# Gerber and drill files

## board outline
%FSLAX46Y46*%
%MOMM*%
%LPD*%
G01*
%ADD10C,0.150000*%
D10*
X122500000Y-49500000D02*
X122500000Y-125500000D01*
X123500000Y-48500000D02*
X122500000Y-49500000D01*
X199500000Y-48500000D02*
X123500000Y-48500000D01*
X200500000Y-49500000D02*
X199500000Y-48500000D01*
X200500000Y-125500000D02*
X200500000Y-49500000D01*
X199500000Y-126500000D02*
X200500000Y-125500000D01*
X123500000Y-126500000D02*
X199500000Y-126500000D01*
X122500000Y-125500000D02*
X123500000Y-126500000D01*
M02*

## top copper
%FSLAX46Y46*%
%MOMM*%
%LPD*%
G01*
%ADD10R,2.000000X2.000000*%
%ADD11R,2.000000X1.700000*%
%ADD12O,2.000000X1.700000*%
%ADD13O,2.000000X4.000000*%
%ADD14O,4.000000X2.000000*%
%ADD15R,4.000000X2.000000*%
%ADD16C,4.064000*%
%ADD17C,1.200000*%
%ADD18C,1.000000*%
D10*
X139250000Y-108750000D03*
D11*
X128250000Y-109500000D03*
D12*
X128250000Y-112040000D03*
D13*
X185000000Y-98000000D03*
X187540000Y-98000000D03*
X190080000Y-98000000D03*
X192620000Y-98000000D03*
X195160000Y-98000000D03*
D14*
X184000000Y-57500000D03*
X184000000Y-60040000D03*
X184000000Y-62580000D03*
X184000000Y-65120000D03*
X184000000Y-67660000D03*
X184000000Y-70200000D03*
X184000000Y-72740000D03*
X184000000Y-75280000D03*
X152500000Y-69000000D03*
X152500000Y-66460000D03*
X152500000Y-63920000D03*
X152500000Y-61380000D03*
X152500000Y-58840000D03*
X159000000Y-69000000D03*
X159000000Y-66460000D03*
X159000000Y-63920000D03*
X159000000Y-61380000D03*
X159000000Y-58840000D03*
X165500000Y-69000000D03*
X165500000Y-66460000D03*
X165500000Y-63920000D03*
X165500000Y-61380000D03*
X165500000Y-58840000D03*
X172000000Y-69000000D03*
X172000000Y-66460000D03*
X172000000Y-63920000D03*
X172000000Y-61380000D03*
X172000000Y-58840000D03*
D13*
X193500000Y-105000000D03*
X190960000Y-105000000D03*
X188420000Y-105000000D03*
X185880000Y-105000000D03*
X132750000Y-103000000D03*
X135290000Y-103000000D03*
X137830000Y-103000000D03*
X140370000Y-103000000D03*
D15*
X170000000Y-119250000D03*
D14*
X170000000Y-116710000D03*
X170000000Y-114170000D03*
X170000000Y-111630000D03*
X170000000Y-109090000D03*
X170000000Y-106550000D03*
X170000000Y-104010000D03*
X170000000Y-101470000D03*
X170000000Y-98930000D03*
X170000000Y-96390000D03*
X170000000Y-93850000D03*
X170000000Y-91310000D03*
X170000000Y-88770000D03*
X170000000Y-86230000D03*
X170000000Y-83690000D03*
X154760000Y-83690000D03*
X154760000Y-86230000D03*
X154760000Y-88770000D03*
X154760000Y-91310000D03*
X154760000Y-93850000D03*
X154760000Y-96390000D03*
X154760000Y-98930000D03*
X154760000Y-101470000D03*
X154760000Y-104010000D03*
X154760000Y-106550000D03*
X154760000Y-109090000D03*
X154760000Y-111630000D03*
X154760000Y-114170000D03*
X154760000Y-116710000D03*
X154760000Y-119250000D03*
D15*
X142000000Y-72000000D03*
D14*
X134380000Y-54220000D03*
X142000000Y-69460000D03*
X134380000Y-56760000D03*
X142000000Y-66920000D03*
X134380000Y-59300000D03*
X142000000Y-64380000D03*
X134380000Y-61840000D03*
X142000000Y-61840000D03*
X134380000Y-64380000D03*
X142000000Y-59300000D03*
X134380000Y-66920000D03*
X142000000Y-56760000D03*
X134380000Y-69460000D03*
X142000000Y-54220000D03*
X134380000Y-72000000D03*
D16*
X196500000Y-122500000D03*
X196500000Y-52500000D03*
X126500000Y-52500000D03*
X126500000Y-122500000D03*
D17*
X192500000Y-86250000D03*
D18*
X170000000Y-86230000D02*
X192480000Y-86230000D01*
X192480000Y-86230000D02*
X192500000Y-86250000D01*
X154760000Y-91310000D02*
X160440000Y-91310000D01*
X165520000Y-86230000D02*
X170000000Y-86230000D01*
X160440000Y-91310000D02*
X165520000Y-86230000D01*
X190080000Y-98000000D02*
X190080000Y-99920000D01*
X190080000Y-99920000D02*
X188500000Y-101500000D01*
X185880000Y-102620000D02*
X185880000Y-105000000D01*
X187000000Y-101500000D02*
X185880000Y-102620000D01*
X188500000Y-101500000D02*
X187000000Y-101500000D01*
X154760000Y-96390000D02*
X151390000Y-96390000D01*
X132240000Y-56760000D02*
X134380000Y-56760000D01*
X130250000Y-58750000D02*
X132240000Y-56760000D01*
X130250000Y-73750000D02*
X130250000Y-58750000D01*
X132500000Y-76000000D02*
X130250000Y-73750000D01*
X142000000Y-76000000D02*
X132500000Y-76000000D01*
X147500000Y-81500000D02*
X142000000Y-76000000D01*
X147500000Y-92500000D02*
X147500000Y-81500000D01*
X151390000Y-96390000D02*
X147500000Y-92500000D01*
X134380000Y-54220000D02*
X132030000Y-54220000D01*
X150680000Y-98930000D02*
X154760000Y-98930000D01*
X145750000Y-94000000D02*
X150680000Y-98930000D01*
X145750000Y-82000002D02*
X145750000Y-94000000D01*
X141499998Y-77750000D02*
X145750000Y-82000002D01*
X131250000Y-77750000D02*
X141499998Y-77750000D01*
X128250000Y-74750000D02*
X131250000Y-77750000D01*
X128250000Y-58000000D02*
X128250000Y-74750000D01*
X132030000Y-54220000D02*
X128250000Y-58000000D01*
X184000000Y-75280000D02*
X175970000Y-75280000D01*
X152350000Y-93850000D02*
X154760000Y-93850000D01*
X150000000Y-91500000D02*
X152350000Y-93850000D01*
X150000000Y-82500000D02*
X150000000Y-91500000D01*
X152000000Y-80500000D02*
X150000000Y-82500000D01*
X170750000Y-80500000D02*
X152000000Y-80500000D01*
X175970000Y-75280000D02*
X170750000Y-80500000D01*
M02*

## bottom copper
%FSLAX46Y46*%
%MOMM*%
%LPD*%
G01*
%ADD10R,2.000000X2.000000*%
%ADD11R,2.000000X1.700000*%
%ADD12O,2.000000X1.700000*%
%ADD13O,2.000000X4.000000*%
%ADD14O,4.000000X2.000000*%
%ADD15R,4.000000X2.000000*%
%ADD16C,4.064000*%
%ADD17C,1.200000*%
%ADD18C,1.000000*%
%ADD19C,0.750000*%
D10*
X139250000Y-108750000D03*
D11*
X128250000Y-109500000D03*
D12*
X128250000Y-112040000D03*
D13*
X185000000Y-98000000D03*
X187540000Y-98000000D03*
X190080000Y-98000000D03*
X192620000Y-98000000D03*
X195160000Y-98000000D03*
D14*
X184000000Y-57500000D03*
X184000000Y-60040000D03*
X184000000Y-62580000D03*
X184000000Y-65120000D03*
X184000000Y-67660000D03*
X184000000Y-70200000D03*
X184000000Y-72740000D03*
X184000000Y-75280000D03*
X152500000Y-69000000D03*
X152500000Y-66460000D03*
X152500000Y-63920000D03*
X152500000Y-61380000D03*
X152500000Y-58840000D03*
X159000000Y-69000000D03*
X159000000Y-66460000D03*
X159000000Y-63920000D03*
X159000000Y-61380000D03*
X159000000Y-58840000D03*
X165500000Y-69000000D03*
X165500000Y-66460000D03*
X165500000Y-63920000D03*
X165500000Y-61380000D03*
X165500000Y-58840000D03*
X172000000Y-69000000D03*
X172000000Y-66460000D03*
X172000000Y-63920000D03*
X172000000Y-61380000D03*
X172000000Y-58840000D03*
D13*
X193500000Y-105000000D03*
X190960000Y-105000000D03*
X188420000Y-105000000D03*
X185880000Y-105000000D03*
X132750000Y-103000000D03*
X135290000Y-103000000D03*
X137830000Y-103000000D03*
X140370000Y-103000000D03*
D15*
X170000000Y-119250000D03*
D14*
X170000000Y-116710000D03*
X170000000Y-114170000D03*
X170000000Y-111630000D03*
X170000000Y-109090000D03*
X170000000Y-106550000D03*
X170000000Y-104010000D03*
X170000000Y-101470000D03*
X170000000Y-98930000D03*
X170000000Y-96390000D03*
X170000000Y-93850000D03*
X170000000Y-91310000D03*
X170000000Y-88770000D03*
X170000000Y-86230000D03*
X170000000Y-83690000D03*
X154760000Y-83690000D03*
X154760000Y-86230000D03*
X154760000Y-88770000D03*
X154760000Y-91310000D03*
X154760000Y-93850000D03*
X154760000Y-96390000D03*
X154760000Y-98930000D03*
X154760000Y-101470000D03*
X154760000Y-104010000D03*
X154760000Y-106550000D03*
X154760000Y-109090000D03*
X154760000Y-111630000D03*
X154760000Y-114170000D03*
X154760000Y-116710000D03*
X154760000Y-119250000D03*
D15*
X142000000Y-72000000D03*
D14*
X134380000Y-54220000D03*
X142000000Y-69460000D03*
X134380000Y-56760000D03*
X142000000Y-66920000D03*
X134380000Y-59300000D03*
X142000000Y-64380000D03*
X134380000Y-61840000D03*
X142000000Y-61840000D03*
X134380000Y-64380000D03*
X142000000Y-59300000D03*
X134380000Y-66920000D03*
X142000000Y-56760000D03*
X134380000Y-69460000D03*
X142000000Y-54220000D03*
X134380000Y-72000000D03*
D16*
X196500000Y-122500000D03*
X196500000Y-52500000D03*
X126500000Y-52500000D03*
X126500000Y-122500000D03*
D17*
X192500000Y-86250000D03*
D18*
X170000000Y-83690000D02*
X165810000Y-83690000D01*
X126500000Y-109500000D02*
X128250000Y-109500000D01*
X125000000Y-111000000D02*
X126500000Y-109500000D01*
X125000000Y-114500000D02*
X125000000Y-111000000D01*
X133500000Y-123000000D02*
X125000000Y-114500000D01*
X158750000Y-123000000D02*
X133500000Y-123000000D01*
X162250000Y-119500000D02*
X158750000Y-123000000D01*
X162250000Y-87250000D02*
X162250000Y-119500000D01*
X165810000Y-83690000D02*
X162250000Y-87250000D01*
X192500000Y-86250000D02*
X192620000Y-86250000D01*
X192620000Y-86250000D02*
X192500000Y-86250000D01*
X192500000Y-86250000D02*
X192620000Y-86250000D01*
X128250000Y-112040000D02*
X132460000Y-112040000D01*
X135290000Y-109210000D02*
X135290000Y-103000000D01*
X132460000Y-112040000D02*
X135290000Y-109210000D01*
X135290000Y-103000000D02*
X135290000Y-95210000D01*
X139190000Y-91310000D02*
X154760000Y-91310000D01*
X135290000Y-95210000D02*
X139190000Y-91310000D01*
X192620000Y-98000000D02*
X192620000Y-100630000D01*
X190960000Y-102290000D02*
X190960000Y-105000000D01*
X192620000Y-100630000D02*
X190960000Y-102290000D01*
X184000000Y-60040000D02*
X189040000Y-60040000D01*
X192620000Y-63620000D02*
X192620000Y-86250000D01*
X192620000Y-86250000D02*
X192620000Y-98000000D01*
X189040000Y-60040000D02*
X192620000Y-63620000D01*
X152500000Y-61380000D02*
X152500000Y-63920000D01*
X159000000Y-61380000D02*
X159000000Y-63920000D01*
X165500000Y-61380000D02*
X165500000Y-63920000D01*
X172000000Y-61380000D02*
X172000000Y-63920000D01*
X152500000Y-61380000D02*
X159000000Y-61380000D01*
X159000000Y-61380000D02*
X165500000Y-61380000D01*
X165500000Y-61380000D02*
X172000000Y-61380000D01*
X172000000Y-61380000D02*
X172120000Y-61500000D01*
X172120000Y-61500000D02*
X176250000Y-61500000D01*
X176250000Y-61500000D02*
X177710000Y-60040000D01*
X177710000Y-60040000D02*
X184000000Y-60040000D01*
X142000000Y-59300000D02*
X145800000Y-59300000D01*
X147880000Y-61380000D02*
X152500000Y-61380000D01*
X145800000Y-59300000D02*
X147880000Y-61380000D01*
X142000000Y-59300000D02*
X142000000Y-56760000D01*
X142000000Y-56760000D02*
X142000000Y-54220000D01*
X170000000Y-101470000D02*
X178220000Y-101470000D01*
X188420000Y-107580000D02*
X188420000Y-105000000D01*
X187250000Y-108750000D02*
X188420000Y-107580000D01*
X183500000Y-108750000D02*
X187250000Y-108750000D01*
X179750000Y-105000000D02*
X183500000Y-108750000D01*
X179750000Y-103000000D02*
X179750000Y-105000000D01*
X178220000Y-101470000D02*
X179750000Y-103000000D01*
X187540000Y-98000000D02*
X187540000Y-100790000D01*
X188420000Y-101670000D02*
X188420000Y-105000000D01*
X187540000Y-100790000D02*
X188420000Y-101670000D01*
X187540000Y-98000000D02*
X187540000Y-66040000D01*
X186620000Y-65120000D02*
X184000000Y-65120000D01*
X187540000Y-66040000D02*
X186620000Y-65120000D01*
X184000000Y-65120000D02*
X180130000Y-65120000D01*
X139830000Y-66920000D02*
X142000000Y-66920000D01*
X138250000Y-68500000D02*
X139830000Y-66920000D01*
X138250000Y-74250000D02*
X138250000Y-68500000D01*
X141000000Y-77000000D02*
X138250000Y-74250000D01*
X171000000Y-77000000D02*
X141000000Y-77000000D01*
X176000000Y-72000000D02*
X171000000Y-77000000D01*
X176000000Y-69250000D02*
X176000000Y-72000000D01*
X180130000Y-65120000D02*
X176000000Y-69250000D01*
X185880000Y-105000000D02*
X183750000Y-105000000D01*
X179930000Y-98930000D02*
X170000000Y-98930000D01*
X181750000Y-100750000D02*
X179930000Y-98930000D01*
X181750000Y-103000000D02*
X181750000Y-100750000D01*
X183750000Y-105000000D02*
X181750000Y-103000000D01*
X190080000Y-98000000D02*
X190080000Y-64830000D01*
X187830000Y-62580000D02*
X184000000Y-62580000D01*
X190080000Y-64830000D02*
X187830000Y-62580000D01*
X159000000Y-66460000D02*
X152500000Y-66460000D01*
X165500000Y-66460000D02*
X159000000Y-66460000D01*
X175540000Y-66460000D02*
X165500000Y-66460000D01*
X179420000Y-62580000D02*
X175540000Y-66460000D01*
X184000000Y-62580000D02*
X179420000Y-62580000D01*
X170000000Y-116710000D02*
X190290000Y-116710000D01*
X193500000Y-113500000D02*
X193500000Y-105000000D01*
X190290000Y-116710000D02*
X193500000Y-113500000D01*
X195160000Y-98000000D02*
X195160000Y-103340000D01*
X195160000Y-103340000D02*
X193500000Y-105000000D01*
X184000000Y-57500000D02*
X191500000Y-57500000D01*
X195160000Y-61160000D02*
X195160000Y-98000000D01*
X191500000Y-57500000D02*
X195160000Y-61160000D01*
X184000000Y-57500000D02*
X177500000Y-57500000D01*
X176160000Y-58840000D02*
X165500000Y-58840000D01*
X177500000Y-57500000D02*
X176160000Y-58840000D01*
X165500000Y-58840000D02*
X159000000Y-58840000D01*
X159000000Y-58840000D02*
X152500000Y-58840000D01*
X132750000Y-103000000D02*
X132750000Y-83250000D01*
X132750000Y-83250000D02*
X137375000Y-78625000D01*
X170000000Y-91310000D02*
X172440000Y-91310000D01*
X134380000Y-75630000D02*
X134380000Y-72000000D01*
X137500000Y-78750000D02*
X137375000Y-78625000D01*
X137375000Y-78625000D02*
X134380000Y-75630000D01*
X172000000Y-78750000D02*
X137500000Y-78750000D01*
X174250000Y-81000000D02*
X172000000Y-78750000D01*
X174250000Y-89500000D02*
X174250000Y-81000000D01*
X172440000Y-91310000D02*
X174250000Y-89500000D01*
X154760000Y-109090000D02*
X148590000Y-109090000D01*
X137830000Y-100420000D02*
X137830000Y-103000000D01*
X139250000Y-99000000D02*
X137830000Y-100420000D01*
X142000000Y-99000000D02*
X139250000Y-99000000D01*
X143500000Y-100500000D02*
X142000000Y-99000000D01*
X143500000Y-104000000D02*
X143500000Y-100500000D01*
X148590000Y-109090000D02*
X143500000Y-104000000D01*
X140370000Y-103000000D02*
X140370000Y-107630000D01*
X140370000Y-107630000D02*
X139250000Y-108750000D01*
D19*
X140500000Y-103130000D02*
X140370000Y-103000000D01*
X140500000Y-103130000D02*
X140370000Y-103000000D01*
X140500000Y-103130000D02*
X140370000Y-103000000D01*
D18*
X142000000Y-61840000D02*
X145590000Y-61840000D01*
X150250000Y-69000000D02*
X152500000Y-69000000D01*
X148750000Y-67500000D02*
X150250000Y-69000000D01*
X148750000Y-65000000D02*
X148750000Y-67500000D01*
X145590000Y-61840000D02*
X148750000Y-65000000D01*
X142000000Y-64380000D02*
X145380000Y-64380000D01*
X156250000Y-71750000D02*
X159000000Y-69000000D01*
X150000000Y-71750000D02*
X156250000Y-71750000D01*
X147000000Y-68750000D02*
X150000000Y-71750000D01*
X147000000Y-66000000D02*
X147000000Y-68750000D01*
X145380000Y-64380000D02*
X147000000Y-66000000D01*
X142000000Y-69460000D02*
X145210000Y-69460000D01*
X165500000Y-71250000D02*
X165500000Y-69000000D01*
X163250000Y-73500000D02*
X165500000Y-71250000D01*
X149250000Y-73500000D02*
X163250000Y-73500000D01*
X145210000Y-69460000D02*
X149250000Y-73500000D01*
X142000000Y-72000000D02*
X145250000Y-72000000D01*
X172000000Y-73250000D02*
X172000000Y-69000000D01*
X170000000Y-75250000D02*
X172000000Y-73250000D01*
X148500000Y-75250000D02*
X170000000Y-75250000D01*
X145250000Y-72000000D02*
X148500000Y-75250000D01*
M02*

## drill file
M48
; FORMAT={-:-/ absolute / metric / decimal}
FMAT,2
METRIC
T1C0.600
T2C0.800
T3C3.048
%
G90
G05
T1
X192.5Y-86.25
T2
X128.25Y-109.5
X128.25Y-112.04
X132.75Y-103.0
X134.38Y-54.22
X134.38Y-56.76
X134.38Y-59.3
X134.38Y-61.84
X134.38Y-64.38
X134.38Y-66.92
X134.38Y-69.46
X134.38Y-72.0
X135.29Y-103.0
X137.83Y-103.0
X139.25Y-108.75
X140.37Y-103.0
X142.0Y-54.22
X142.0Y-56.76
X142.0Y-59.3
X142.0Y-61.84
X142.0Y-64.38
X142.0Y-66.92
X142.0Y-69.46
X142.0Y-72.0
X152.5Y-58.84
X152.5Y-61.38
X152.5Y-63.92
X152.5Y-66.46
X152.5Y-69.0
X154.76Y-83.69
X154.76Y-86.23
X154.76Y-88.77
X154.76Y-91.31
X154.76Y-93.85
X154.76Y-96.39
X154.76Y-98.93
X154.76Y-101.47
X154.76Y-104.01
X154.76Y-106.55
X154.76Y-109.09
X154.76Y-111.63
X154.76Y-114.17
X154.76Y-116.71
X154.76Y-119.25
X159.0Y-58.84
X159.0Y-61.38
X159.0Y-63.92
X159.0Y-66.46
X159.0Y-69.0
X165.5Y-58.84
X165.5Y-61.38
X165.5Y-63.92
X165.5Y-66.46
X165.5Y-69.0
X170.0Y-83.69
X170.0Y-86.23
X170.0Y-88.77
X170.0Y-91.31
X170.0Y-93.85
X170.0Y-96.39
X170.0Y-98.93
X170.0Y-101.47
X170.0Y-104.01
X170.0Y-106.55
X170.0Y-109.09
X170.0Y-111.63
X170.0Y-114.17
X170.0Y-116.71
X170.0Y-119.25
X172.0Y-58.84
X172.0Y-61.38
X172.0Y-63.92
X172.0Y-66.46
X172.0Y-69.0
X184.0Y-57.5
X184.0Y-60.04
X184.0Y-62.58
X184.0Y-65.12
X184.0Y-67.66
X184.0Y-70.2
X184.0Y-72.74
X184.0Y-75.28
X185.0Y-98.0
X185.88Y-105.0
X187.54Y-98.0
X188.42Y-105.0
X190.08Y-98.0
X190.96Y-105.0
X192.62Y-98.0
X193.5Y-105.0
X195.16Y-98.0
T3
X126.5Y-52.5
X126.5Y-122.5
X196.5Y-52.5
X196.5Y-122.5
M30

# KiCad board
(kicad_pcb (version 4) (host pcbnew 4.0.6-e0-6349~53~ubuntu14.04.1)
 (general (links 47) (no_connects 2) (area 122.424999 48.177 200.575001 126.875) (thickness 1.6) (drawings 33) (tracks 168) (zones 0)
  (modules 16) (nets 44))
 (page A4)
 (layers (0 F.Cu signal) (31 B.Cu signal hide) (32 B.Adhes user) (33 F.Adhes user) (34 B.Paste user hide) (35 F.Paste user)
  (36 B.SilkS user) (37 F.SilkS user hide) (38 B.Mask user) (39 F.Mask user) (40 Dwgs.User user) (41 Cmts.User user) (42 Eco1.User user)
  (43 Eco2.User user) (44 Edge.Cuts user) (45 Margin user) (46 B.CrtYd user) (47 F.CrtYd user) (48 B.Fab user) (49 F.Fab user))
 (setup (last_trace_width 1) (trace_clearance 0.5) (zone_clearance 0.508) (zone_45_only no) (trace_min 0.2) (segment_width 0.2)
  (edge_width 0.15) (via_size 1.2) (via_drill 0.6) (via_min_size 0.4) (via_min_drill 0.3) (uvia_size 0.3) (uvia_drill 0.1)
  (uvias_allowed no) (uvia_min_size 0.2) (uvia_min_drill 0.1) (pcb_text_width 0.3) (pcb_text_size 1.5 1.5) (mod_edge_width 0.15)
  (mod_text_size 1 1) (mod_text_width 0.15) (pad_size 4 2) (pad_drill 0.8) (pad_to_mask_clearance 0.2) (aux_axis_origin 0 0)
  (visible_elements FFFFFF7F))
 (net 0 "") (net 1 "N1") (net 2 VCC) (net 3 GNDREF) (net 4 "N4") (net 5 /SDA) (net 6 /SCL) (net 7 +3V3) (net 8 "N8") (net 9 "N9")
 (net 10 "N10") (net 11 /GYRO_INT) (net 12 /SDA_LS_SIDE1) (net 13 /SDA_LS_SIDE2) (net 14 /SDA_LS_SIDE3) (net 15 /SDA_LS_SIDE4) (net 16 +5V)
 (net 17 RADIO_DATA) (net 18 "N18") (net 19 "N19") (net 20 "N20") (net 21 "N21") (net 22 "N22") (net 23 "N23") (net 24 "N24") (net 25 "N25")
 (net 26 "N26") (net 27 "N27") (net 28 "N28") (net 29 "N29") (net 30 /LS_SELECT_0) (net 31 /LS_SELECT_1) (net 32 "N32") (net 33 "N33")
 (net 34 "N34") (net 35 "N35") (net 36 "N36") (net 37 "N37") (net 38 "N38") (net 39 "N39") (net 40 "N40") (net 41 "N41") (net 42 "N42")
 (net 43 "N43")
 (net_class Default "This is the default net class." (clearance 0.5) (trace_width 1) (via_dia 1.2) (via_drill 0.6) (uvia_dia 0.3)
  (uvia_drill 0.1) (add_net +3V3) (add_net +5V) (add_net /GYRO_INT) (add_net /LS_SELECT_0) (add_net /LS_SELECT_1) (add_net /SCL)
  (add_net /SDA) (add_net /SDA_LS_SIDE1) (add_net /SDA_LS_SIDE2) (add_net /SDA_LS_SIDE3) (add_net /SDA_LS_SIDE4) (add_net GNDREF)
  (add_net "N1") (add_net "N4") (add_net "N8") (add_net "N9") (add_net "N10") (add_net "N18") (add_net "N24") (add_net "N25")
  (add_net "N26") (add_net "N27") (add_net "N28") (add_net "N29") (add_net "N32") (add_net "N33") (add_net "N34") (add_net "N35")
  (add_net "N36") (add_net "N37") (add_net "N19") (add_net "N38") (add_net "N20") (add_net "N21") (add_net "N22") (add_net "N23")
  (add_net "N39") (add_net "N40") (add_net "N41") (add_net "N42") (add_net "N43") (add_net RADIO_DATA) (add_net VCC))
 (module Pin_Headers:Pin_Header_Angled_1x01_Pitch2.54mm (layer F.Cu) (at 139.25 108.75 270)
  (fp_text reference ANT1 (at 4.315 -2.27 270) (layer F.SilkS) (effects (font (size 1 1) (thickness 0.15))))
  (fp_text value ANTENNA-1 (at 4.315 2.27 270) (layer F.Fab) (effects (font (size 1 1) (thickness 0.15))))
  (pad 1 thru_hole rect (at 0 0 270) (size 2 2) (drill 0.8) (layers *.Cu *.Mask) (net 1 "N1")))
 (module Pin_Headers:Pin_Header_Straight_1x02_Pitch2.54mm (layer F.Cu) (at 128.25 109.5)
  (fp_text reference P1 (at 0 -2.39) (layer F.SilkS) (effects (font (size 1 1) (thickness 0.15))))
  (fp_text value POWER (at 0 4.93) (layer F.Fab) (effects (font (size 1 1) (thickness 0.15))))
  (pad 1 thru_hole rect (at 0 0) (size 2 1.7) (drill 0.8) (layers *.Cu *.Mask) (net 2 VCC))
  (pad 2 thru_hole oval (at 0 2.54) (size 2 1.7) (drill 0.8) (layers *.Cu *.Mask) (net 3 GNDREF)))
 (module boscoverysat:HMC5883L (layer F.Cu) (at 185 98)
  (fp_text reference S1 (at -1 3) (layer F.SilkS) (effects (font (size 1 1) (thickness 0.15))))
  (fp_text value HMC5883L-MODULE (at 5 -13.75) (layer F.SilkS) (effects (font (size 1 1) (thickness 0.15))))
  (pad 1 thru_hole oval (at 0 0) (size 2 4) (drill 0.8) (layers *.Cu F.SilkS B.Mask) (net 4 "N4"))
  (pad 2 thru_hole oval (at 2.54 0) (size 2 4) (drill 0.8) (layers *.Cu F.SilkS B.Mask) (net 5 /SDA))
  (pad 3 thru_hole oval (at 5.08 0) (size 2 4) (drill 0.8) (layers *.Cu F.SilkS B.Mask) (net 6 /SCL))
  (pad 4 thru_hole oval (at 7.62 0) (size 2 4) (drill 0.8) (layers *.Cu F.SilkS B.Mask) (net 3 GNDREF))
  (pad 5 thru_hole oval (at 10.16 0) (size 2 4) (drill 0.8) (layers *.Cu F.SilkS B.Mask) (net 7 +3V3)))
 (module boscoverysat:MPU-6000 (layer F.Cu) (at 184 57.5 270)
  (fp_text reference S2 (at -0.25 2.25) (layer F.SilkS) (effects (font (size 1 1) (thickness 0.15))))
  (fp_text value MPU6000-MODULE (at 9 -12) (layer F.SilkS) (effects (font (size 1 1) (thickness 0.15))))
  (pad 1 thru_hole oval (at 0 0 270) (size 2 4) (drill 0.8) (layers *.Cu F.SilkS B.Mask) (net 7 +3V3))
  (pad 2 thru_hole oval (at 2.54 0 270) (size 2 4) (drill 0.8) (layers *.Cu F.SilkS B.Mask) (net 3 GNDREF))
  (pad 3 thru_hole oval (at 5.08 0 270) (size 2 4) (drill 0.8) (layers *.Cu F.SilkS B.Mask) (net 6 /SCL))
  (pad 4 thru_hole oval (at 7.62 0 270) (size 2 4) (drill 0.8) (layers *.Cu F.SilkS B.Mask) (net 5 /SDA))
  (pad 5 thru_hole oval (at 10.16 0 270) (size 2 4) (drill 0.8) (layers *.Cu F.SilkS B.Mask) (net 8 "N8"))
  (pad 6 thru_hole oval (at 12.7 0 270) (size 2 4) (drill 0.8) (layers *.Cu F.SilkS B.Mask) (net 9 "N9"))
  (pad 7 thru_hole oval (at 15.24 0 270) (size 2 4) (drill 0.8) (layers *.Cu F.SilkS B.Mask) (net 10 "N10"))
  (pad 8 thru_hole oval (at 17.78 0 270) (size 2 4) (drill 0.8) (layers *.Cu F.SilkS B.Mask) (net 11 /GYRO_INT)))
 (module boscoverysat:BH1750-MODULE (layer F.Cu) (at 152.5 69 90)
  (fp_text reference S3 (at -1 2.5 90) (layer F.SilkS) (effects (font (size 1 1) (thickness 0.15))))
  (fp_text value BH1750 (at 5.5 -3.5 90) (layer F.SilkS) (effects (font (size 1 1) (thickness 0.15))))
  (pad 1 thru_hole oval (at 0 0 90) (size 2 4) (drill 0.8) (layers *.Cu F.SilkS B.Mask) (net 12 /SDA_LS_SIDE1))
  (pad 2 thru_hole oval (at 2.54 0 90) (size 2 4) (drill 0.8) (layers *.Cu F.SilkS B.Mask) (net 6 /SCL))
  (pad 3 thru_hole oval (at 5.08 0 90) (size 2 4) (drill 0.8) (layers *.Cu F.SilkS B.Mask) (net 3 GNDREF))
  (pad 4 thru_hole oval (at 7.62 0 90) (size 2 4) (drill 0.8) (layers *.Cu F.SilkS B.Mask) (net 3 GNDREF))
  (pad 5 thru_hole oval (at 10.16 0 90) (size 2 4) (drill 0.8) (layers *.Cu F.SilkS B.Mask) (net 7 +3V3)))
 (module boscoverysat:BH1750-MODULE (layer F.Cu) (at 159 69 90)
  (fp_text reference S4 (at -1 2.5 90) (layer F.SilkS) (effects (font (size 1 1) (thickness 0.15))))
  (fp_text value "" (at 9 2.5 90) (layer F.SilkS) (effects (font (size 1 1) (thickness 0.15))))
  (pad 1 thru_hole oval (at 0 0 90) (size 2 4) (drill 0.8) (layers *.Cu F.SilkS B.Mask) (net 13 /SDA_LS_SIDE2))
  (pad 2 thru_hole oval (at 2.54 0 90) (size 2 4) (drill 0.8) (layers *.Cu F.SilkS B.Mask) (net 6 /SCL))
  (pad 3 thru_hole oval (at 5.08 0 90) (size 2 4) (drill 0.8) (layers *.Cu F.SilkS B.Mask) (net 3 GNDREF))
  (pad 4 thru_hole oval (at 7.62 0 90) (size 2 4) (drill 0.8) (layers *.Cu F.SilkS B.Mask) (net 3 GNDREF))
  (pad 5 thru_hole oval (at 10.16 0 90) (size 2 4) (drill 0.8) (layers *.Cu F.SilkS B.Mask) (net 7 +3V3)))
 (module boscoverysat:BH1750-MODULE (layer F.Cu) (at 165.5 69 90)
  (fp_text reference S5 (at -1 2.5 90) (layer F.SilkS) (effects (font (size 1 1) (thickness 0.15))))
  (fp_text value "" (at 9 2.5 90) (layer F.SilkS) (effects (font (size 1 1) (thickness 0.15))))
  (pad 1 thru_hole oval (at 0 0 90) (size 2 4) (drill 0.8) (layers *.Cu F.SilkS B.Mask) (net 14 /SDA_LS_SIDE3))
  (pad 2 thru_hole oval (at 2.54 0 90) (size 2 4) (drill 0.8) (layers *.Cu F.SilkS B.Mask) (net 6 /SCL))
  (pad 3 thru_hole oval (at 5.08 0 90) (size 2 4) (drill 0.8) (layers *.Cu F.SilkS B.Mask) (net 3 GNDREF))
  (pad 4 thru_hole oval (at 7.62 0 90) (size 2 4) (drill 0.8) (layers *.Cu F.SilkS B.Mask) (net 3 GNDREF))
  (pad 5 thru_hole oval (at 10.16 0 90) (size 2 4) (drill 0.8) (layers *.Cu F.SilkS B.Mask) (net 7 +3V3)))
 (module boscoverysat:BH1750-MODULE (layer F.Cu) (at 172 69 90)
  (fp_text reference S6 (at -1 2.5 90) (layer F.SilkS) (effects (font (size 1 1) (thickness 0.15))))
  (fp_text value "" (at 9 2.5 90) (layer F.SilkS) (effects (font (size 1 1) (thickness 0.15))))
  (pad 1 thru_hole oval (at 0 0 90) (size 2 4) (drill 0.8) (layers *.Cu F.SilkS B.Mask) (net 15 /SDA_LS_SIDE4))
  (pad 2 thru_hole oval (at 2.54 0 90) (size 2 4) (drill 0.8) (layers *.Cu F.SilkS B.Mask) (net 6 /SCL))
  (pad 3 thru_hole oval (at 5.08 0 90) (size 2 4) (drill 0.8) (layers *.Cu F.SilkS B.Mask) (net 3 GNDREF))
  (pad 4 thru_hole oval (at 7.62 0 90) (size 2 4) (drill 0.8) (layers *.Cu F.SilkS B.Mask) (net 3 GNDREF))
  (pad 5 thru_hole oval (at 10.16 0 90) (size 2 4) (drill 0.8) (layers *.Cu F.SilkS B.Mask) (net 7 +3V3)))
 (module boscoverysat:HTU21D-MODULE (layer F.Cu) (at 193.5 105 180)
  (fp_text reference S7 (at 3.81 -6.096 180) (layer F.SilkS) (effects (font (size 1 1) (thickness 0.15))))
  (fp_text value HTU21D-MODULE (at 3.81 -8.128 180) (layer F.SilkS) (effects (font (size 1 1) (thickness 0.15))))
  (pad 1 thru_hole oval (at 0 0 180) (size 2 4) (drill 0.8) (layers *.Cu B.Mask) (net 7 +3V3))
  (pad 2 thru_hole oval (at 2.54 0 180) (size 2 4) (drill 0.8) (layers *.Cu B.Mask) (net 3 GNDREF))
  (pad 3 thru_hole oval (at 5.08 0 180) (size 2 4) (drill 0.8) (layers *.Cu B.Mask) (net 5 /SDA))
  (pad 4 thru_hole oval (at 7.62 0 180) (size 2 4) (drill 0.8) (layers *.Cu B.Mask) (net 6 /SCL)))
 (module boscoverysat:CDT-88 (layer F.Cu) (at 132.75 103)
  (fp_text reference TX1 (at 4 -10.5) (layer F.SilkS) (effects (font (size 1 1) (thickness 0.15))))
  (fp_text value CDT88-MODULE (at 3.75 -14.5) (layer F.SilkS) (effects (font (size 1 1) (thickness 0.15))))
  (pad 1 thru_hole oval (at 0 0) (size 2 4) (drill 0.8) (layers *.Cu B.Mask) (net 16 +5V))
  (pad 2 thru_hole oval (at 2.54 0) (size 2 4) (drill 0.8) (layers *.Cu B.Mask) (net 3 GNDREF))
  (pad 3 thru_hole oval (at 5.08 0) (size 2 4) (drill 0.8) (layers *.Cu B.Mask) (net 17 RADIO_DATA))
  (pad 4 thru_hole oval (at 7.62 0) (size 2 4) (drill 0.8) (layers *.Cu B.Mask) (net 1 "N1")))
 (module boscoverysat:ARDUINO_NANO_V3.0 (layer F.Cu) (at 170 119.25 180)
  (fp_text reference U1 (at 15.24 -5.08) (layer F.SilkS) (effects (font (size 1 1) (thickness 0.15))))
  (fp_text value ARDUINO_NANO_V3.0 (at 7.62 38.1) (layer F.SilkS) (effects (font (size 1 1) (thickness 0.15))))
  (pad 1 thru_hole rect (at 0 0 180) (size 4 2) (drill 0.8) (layers *.Cu *.Mask) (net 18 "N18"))
  (pad 2 thru_hole oval (at 0 2.54 180) (size 4 2) (drill 0.8) (layers *.Cu B.Mask) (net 7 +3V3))
  (pad 3 thru_hole oval (at 0 5.08 180) (size 4 2) (drill 0.8) (layers *.Cu B.Mask) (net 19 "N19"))
  (pad 4 thru_hole oval (at 0 7.62 180) (size 4 2) (drill 0.8) (layers *.Cu B.Mask) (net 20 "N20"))
  (pad 5 thru_hole oval (at 0 10.16 180) (size 4 2) (drill 0.8) (layers *.Cu B.Mask) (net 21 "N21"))
  (pad 6 thru_hole oval (at 0 12.7 180) (size 4 2) (drill 0.8) (layers *.Cu B.Mask) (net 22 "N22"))
  (pad 7 thru_hole oval (at 0 15.24 180) (size 4 2) (drill 0.8) (layers *.Cu B.Mask) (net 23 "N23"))
  (pad 8 thru_hole oval (at 0 17.78 180) (size 4 2) (drill 0.8) (layers *.Cu B.Mask) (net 5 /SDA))
  (pad 9 thru_hole oval (at 0 20.32 180) (size 4 2) (drill 0.8) (layers *.Cu B.Mask) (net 6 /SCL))
  (pad 10 thru_hole oval (at 0 22.86 180) (size 4 2) (drill 0.8) (layers *.Cu B.Mask) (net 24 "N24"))
  (pad 11 thru_hole oval (at 0 25.4 180) (size 4 2) (drill 0.8) (layers *.Cu B.Mask) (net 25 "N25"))
  (pad 12 thru_hole oval (at 0 27.94 180) (size 4 2) (drill 0.8) (layers *.Cu B.Mask) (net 16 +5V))
  (pad 13 thru_hole oval (at 0 30.48 180) (size 4 2) (drill 0.8) (layers *.Cu B.Mask) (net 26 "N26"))
  (pad 14 thru_hole oval (at 0 33.02 180) (size 4 2) (drill 0.8) (layers *.Cu B.Mask) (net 3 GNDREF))
  (pad 15 thru_hole oval (at 0 35.56 180) (size 4 2) (drill 0.8) (layers *.Cu B.Mask) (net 2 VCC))
  (pad 16 thru_hole oval (at 15.24 35.56 180) (size 4 2) (drill 0.8) (layers *.Cu B.Mask) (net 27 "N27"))
  (pad 17 thru_hole oval (at 15.24 33.02 180) (size 4 2) (drill 0.8) (layers *.Cu B.Mask) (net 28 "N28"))
  (pad 18 thru_hole oval (at 15.24 30.48 180) (size 4 2) (drill 0.8) (layers *.Cu B.Mask) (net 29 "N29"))
  (pad 19 thru_hole oval (at 15.24 27.94 180) (size 4 2) (drill 0.8) (layers *.Cu B.Mask) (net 3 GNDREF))
  (pad 20 thru_hole oval (at 15.24 25.4 180) (size 4 2) (drill 0.8) (layers *.Cu B.Mask) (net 11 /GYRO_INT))
  (pad 21 thru_hole oval (at 15.24 22.86 180) (size 4 2) (drill 0.8) (layers *.Cu B.Mask) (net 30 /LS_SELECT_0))
  (pad 22 thru_hole oval (at 15.24 20.32 180) (size 4 2) (drill 0.8) (layers *.Cu B.Mask) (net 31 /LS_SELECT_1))
  (pad 23 thru_hole oval (at 15.24 17.78 180) (size 4 2) (drill 0.8) (layers *.Cu B.Mask) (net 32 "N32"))
  (pad 24 thru_hole oval (at 15.24 15.24 180) (size 4 2) (drill 0.8) (layers *.Cu B.Mask) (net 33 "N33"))
  (pad 25 thru_hole oval (at 15.24 12.7 180) (size 4 2) (drill 0.8) (layers *.Cu B.Mask) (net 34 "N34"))
  (pad 26 thru_hole oval (at 15.24 10.16 180) (size 4 2) (drill 0.8) (layers *.Cu B.Mask) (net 17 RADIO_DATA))
  (pad 27 thru_hole oval (at 15.24 7.62 180) (size 4 2) (drill 0.8) (layers *.Cu B.Mask) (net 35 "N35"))
  (pad 28 thru_hole oval (at 15.24 5.08 180) (size 4 2) (drill 0.8) (layers *.Cu B.Mask) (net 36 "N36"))
  (pad 29 thru_hole oval (at 15.24 2.54 180) (size 4 2) (drill 0.8) (layers *.Cu B.Mask) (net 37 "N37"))
  (pad 30 thru_hole oval (at 15.24 0 180) (size 4 2) (drill 0.8) (layers *.Cu B.Mask) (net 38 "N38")))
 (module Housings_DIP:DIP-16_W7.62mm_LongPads (layer F.Cu) (at 142 72 180)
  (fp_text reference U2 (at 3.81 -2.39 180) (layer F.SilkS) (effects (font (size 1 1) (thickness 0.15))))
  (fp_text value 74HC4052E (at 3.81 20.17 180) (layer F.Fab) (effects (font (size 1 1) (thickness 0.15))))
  (pad 1 thru_hole rect (at 0 0 180) (size 4 2) (drill 0.8) (layers *.Cu *.Mask) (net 15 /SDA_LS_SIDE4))
  (pad 9 thru_hole oval (at 7.62 17.78 180) (size 4 2) (drill 0.8) (layers *.Cu *.Mask) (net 31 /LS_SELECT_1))
  (pad 2 thru_hole oval (at 0 2.54 180) (size 4 2) (drill 0.8) (layers *.Cu *.Mask) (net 14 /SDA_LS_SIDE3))
  (pad 10 thru_hole oval (at 7.62 15.24 180) (size 4 2) (drill 0.8) (layers *.Cu *.Mask) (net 30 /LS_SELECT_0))
  (pad 3 thru_hole oval (at 0 5.08 180) (size 4 2) (drill 0.8) (layers *.Cu *.Mask) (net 5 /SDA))
  (pad 11 thru_hole oval (at 7.62 12.7 180) (size 4 2) (drill 0.8) (layers *.Cu *.Mask) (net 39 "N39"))
  (pad 4 thru_hole oval (at 0 7.62 180) (size 4 2) (drill 0.8) (layers *.Cu *.Mask) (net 13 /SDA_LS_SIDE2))
  (pad 12 thru_hole oval (at 7.62 10.16 180) (size 4 2) (drill 0.8) (layers *.Cu *.Mask) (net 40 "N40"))
  (pad 5 thru_hole oval (at 0 10.16 180) (size 4 2) (drill 0.8) (layers *.Cu *.Mask) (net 12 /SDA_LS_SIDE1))
  (pad 13 thru_hole oval (at 7.62 7.62 180) (size 4 2) (drill 0.8) (layers *.Cu *.Mask) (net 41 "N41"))
  (pad 6 thru_hole oval (at 0 12.7 180) (size 4 2) (drill 0.8) (layers *.Cu *.Mask) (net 3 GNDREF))
  (pad 14 thru_hole oval (at 7.62 5.08 180) (size 4 2) (drill 0.8) (layers *.Cu *.Mask) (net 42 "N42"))
  (pad 7 thru_hole oval (at 0 15.24 180) (size 4 2) (drill 0.8) (layers *.Cu *.Mask) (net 3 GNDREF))
  (pad 15 thru_hole oval (at 7.62 2.54 180) (size 4 2) (drill 0.8) (layers *.Cu *.Mask) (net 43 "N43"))
  (pad 8 thru_hole oval (at 0 17.78 180) (size 4 2) (drill 0.8) (layers *.Cu *.Mask) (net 3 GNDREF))
  (pad 16 thru_hole oval (at 7.62 0 180) (size 4 2) (drill 0.8) (layers *.Cu *.Mask) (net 16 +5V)))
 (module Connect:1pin (layer F.Cu) (at 196.5 122.5)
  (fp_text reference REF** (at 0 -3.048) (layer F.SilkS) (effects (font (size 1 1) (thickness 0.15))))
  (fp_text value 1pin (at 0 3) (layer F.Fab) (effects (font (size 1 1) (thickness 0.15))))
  (pad 1 thru_hole circle (at 0 0) (size 4.064 4.064) (drill 3.048) (layers *.Cu *.Mask)))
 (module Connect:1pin (layer F.Cu) (at 196.5 52.5)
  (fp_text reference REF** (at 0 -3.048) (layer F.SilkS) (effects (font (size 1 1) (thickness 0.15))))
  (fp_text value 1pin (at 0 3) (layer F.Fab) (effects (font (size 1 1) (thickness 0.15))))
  (pad 1 thru_hole circle (at 0 0) (size 4.064 4.064) (drill 3.048) (layers *.Cu *.Mask)))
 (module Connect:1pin (layer F.Cu) (at 126.5 52.5)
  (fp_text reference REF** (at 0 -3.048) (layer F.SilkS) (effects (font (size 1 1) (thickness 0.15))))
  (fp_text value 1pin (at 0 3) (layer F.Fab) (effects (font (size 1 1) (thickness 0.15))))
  (pad 1 thru_hole circle (at 0 0) (size 4.064 4.064) (drill 3.048) (layers *.Cu *.Mask)))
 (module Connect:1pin (layer F.Cu) (at 126.5 122.5)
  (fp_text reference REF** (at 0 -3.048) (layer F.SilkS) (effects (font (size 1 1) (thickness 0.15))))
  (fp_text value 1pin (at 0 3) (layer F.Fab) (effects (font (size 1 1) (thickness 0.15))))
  (pad 1 thru_hole circle (at 0 0) (size 4.064 4.064) (drill 3.048) (layers *.Cu *.Mask)))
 (gr_line (start 122.5 49.5) (end 122.5 125.5) (angle 90) (layer Edge.Cuts) (width 0.15))
 (gr_line (start 123.5 48.5) (end 122.5 49.5) (angle 90) (layer Edge.Cuts) (width 0.15))
 (gr_line (start 199.5 48.5) (end 123.5 48.5) (angle 90) (layer Edge.Cuts) (width 0.15))
 (gr_line (start 200.5 49.5) (end 199.5 48.5) (angle 90) (layer Edge.Cuts) (width 0.15))
 (gr_line (start 200.5 125.5) (end 200.5 49.5) (angle 90) (layer Edge.Cuts) (width 0.15))
 (gr_line (start 199.5 126.5) (end 200.5 125.5) (angle 90) (layer Edge.Cuts) (width 0.15))
 (gr_line (start 123.5 126.5) (end 199.5 126.5) (angle 90) (layer Edge.Cuts) (width 0.15))
 (gr_line (start 122.5 125.5) (end 123.5 126.5) (angle 90) (layer Edge.Cuts) (width 0.15))
 (segment (start 170 83.69) (end 165.81 83.69) (width 1) (layer B.Cu) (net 2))
 (segment (start 126.5 109.5) (end 128.25 109.5) (width 1) (layer B.Cu) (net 2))
 (segment (start 125 111) (end 126.5 109.5) (width 1) (layer B.Cu) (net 2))
 (segment (start 125 114.5) (end 125 111) (width 1) (layer B.Cu) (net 2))
 (segment (start 133.5 123) (end 125 114.5) (width 1) (layer B.Cu) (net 2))
 (segment (start 158.75 123) (end 133.5 123) (width 1) (layer B.Cu) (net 2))
 (segment (start 162.25 119.5) (end 158.75 123) (width 1) (layer B.Cu) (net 2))
 (segment (start 162.25 87.25) (end 162.25 119.5) (width 1) (layer B.Cu) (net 2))
 (segment (start 165.81 83.69) (end 162.25 87.25) (width 1) (layer B.Cu) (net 2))
 (segment (start 170 86.23) (end 192.48 86.23) (width 1) (layer F.Cu) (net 3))
 (via (at 192.5 86.25) (size 1.2) (drill 0.6) (layers F.Cu B.Cu) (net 3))
 (segment (start 192.48 86.23) (end 192.5 86.25) (width 1) (layer F.Cu) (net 3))
 (segment (start 192.5 86.25) (end 192.62 86.25) (width 1) (layer B.Cu) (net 3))
 (segment (start 192.62 86.25) (end 192.5 86.25) (width 1) (layer B.Cu) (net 3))
 (segment (start 192.5 86.25) (end 192.62 86.25) (width 1) (layer B.Cu) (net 3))
 (segment (start 154.76 91.31) (end 160.44 91.31) (width 1) (layer F.Cu) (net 3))
 (segment (start 165.52 86.23) (end 170 86.23) (width 1) (layer F.Cu) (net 3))
 (segment (start 160.44 91.31) (end 165.52 86.23) (width 1) (layer F.Cu) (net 3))
 (segment (start 128.25 112.04) (end 132.46 112.04) (width 1) (layer B.Cu) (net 3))
 (segment (start 135.29 109.21) (end 135.29 103) (width 1) (layer B.Cu) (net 3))
 (segment (start 132.46 112.04) (end 135.29 109.21) (width 1) (layer B.Cu) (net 3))
 (segment (start 135.29 103) (end 135.29 95.21) (width 1) (layer B.Cu) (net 3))
 (segment (start 139.19 91.31) (end 154.76 91.31) (width 1) (layer B.Cu) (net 3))
 (segment (start 135.29 95.21) (end 139.19 91.31) (width 1) (layer B.Cu) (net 3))
 (segment (start 192.62 98) (end 192.62 100.63) (width 1) (layer B.Cu) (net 3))
 (segment (start 190.96 102.29) (end 190.96 105) (width 1) (layer B.Cu) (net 3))
 (segment (start 192.62 100.63) (end 190.96 102.29) (width 1) (layer B.Cu) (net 3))
 (segment (start 184 60.04) (end 189.04 60.04) (width 1) (layer B.Cu) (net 3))
 (segment (start 192.62 63.62) (end 192.62 86.25) (width 1) (layer B.Cu) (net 3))
 (segment (start 192.62 86.25) (end 192.62 98) (width 1) (layer B.Cu) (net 3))
 (segment (start 189.04 60.04) (end 192.62 63.62) (width 1) (layer B.Cu) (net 3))
 (segment (start 152.5 61.38) (end 152.5 63.92) (width 1) (layer B.Cu) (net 3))
 (segment (start 159 61.38) (end 159 63.92) (width 1) (layer B.Cu) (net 3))
 (segment (start 165.5 61.38) (end 165.5 63.92) (width 1) (layer B.Cu) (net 3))
 (segment (start 172 61.38) (end 172 63.92) (width 1) (layer B.Cu) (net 3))
 (segment (start 152.5 61.38) (end 159 61.38) (width 1) (layer B.Cu) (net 3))
 (segment (start 159 61.38) (end 165.5 61.38) (width 1) (layer B.Cu) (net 3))
 (segment (start 165.5 61.38) (end 172 61.38) (width 1) (layer B.Cu) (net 3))
 (segment (start 172 61.38) (end 172.12 61.5) (width 1) (layer B.Cu) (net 3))
 (segment (start 172.12 61.5) (end 176.25 61.5) (width 1) (layer B.Cu) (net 3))
 (segment (start 176.25 61.5) (end 177.71 60.04) (width 1) (layer B.Cu) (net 3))
 (segment (start 177.71 60.04) (end 184 60.04) (width 1) (layer B.Cu) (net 3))
 (segment (start 142 59.3) (end 145.8 59.3) (width 1) (layer B.Cu) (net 3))
 (segment (start 147.88 61.38) (end 152.5 61.38) (width 1) (layer B.Cu) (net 3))
 (segment (start 145.8 59.3) (end 147.88 61.38) (width 1) (layer B.Cu) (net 3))
 (segment (start 142 59.3) (end 142 56.76) (width 1) (layer B.Cu) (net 3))
 (segment (start 142 56.76) (end 142 54.22) (width 1) (layer B.Cu) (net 3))
 (segment (start 170 101.47) (end 178.22 101.47) (width 1) (layer B.Cu) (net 5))
 (segment (start 188.42 107.58) (end 188.42 105) (width 1) (layer B.Cu) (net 5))
 (segment (start 187.25 108.75) (end 188.42 107.58) (width 1) (layer B.Cu) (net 5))
 (segment (start 183.5 108.75) (end 187.25 108.75) (width 1) (layer B.Cu) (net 5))
 (segment (start 179.75 105) (end 183.5 108.75) (width 1) (layer B.Cu) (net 5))
 (segment (start 179.75 103) (end 179.75 105) (width 1) (layer B.Cu) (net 5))
 (segment (start 178.22 101.47) (end 179.75 103) (width 1) (layer B.Cu) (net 5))
 (segment (start 187.54 98) (end 187.54 100.79) (width 1) (layer B.Cu) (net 5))
 (segment (start 188.42 101.67) (end 188.42 105) (width 1) (layer B.Cu) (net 5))
 (segment (start 187.54 100.79) (end 188.42 101.67) (width 1) (layer B.Cu) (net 5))
 (segment (start 187.54 98) (end 187.54 66.04) (width 1) (layer B.Cu) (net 5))
 (segment (start 186.62 65.12) (end 184 65.12) (width 1) (layer B.Cu) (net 5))
 (segment (start 187.54 66.04) (end 186.62 65.12) (width 1) (layer B.Cu) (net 5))
 (segment (start 184 65.12) (end 180.13 65.12) (width 1) (layer B.Cu) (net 5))
 (segment (start 139.83 66.92) (end 142 66.92) (width 1) (layer B.Cu) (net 5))
 (segment (start 138.25 68.5) (end 139.83 66.92) (width 1) (layer B.Cu) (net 5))
 (segment (start 138.25 74.25) (end 138.25 68.5) (width 1) (layer B.Cu) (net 5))
 (segment (start 141 77) (end 138.25 74.25) (width 1) (layer B.Cu) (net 5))
 (segment (start 171 77) (end 141 77) (width 1) (layer B.Cu) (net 5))
 (segment (start 176 72) (end 171 77) (width 1) (layer B.Cu) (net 5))
 (segment (start 176 69.25) (end 176 72) (width 1) (layer B.Cu) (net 5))
 (segment (start 180.13 65.12) (end 176 69.25) (width 1) (layer B.Cu) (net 5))
 (segment (start 190.08 98) (end 190.08 99.92) (width 1) (layer F.Cu) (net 6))
 (segment (start 190.08 99.92) (end 188.5 101.5) (width 1) (layer F.Cu) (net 6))
 (segment (start 185.88 102.62) (end 185.88 105) (width 1) (layer F.Cu) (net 6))
 (segment (start 187 101.5) (end 185.88 102.62) (width 1) (layer F.Cu) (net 6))
 (segment (start 188.5 101.5) (end 187 101.5) (width 1) (layer F.Cu) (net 6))
 (segment (start 185.88 105) (end 183.75 105) (width 1) (layer B.Cu) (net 6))
 (segment (start 179.93 98.93) (end 170 98.93) (width 1) (layer B.Cu) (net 6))
 (segment (start 181.75 100.75) (end 179.93 98.93) (width 1) (layer B.Cu) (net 6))
 (segment (start 181.75 103) (end 181.75 100.75) (width 1) (layer B.Cu) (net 6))
 (segment (start 183.75 105) (end 181.75 103) (width 1) (layer B.Cu) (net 6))
 (segment (start 190.08 98) (end 190.08 64.83) (width 1) (layer B.Cu) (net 6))
 (segment (start 187.83 62.58) (end 184 62.58) (width 1) (layer B.Cu) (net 6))
 (segment (start 190.08 64.83) (end 187.83 62.58) (width 1) (layer B.Cu) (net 6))
 (segment (start 159 66.46) (end 152.5 66.46) (width 1) (layer B.Cu) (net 6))
 (segment (start 165.5 66.46) (end 159 66.46) (width 1) (layer B.Cu) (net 6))
 (segment (start 175.54 66.46) (end 165.5 66.46) (width 1) (layer B.Cu) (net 6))
 (segment (start 179.42 62.58) (end 175.54 66.46) (width 1) (layer B.Cu) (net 6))
 (segment (start 184 62.58) (end 179.42 62.58) (width 1) (layer B.Cu) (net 6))
 (segment (start 170 116.71) (end 190.29 116.71) (width 1) (layer B.Cu) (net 7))
 (segment (start 193.5 113.5) (end 193.5 105) (width 1) (layer B.Cu) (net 7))
 (segment (start 190.29 116.71) (end 193.5 113.5) (width 1) (layer B.Cu) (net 7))
 (segment (start 195.16 98) (end 195.16 103.34) (width 1) (layer B.Cu) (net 7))
 (segment (start 195.16 103.34) (end 193.5 105) (width 1) (layer B.Cu) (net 7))
 (segment (start 184 57.5) (end 191.5 57.5) (width 1) (layer B.Cu) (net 7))
 (segment (start 195.16 61.16) (end 195.16 98) (width 1) (layer B.Cu) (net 7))
 (segment (start 191.5 57.5) (end 195.16 61.16) (width 1) (layer B.Cu) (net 7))
 (segment (start 184 57.5) (end 177.5 57.5) (width 1) (layer B.Cu) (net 7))
 (segment (start 176.16 58.84) (end 165.5 58.84) (width 1) (layer B.Cu) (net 7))
 (segment (start 177.5 57.5) (end 176.16 58.84) (width 1) (layer B.Cu) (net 7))
 (segment (start 165.5 58.84) (end 159 58.84) (width 1) (layer B.Cu) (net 7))
 (segment (start 159 58.84) (end 152.5 58.84) (width 1) (layer B.Cu) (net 7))
 (segment (start 132.75 103) (end 132.75 83.25) (width 1) (layer B.Cu) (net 16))
 (segment (start 132.75 83.25) (end 137.375 78.625) (width 1) (layer B.Cu) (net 16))
 (segment (start 170 91.31) (end 172.44 91.31) (width 1) (layer B.Cu) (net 16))
 (segment (start 134.38 75.63) (end 134.38 72) (width 1) (layer B.Cu) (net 16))
 (segment (start 137.5 78.75) (end 137.375 78.625) (width 1) (layer B.Cu) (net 16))
 (segment (start 137.375 78.625) (end 134.38 75.63) (width 1) (layer B.Cu) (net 16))
 (segment (start 172 78.75) (end 137.5 78.75) (width 1) (layer B.Cu) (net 16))
 (segment (start 174.25 81) (end 172 78.75) (width 1) (layer B.Cu) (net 16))
 (segment (start 174.25 89.5) (end 174.25 81) (width 1) (layer B.Cu) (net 16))
 (segment (start 172.44 91.31) (end 174.25 89.5) (width 1) (layer B.Cu) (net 16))
 (segment (start 154.76 109.09) (end 148.59 109.09) (width 1) (layer B.Cu) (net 17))
 (segment (start 137.83 100.42) (end 137.83 103) (width 1) (layer B.Cu) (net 17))
 (segment (start 139.25 99) (end 137.83 100.42) (width 1) (layer B.Cu) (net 17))
 (segment (start 142 99) (end 139.25 99) (width 1) (layer B.Cu) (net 17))
 (segment (start 143.5 100.5) (end 142 99) (width 1) (layer B.Cu) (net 17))
 (segment (start 143.5 104) (end 143.5 100.5) (width 1) (layer B.Cu) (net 17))
 (segment (start 148.59 109.09) (end 143.5 104) (width 1) (layer B.Cu) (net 17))
 (segment (start 154.76 96.39) (end 151.39 96.39) (width 1) (layer F.Cu) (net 30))
 (segment (start 132.24 56.76) (end 134.38 56.76) (width 1) (layer F.Cu) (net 30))
 (segment (start 130.25 58.75) (end 132.24 56.76) (width 1) (layer F.Cu) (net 30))
 (segment (start 130.25 73.75) (end 130.25 58.75) (width 1) (layer F.Cu) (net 30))
 (segment (start 132.5 76) (end 130.25 73.75) (width 1) (layer F.Cu) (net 30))
 (segment (start 142 76) (end 132.5 76) (width 1) (layer F.Cu) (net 30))
 (segment (start 147.5 81.5) (end 142 76) (width 1) (layer F.Cu) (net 30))
 (segment (start 147.5 92.5) (end 147.5 81.5) (width 1) (layer F.Cu) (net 30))
 (segment (start 151.39 96.39) (end 147.5 92.5) (width 1) (layer F.Cu) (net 30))
 (segment (start 134.38 54.22) (end 132.03 54.22) (width 1) (layer F.Cu) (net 31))
 (segment (start 150.68 98.93) (end 154.76 98.93) (width 1) (layer F.Cu) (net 31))
 (segment (start 145.75 94) (end 150.68 98.93) (width 1) (layer F.Cu) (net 31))
 (segment (start 145.75 82.000002) (end 145.75 94) (width 1) (layer F.Cu) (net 31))
 (segment (start 141.499998 77.75) (end 145.75 82.000002) (width 1) (layer F.Cu) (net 31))
 (segment (start 131.25 77.75) (end 141.499998 77.75) (width 1) (layer F.Cu) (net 31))
 (segment (start 128.25 74.75) (end 131.25 77.75) (width 1) (layer F.Cu) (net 31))
 (segment (start 128.25 58) (end 128.25 74.75) (width 1) (layer F.Cu) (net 31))
 (segment (start 132.03 54.22) (end 128.25 58) (width 1) (layer F.Cu) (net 31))
 (segment (start 140.37 103) (end 140.37 107.63) (width 1) (layer B.Cu) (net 1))
 (segment (start 140.37 107.63) (end 139.25 108.75) (width 1) (layer B.Cu) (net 1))
 (segment (start 140.5 103.13) (end 140.37 103) (width 0.75) (layer B.Cu) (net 1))
 (segment (start 140.5 103.13) (end 140.37 103) (width 0.75) (layer B.Cu) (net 1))
 (segment (start 140.5 103.13) (end 140.37 103) (width 0.75) (layer B.Cu) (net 1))
 (segment (start 142 61.84) (end 145.59 61.84) (width 1) (layer B.Cu) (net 12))
 (segment (start 150.25 69) (end 152.5 69) (width 1) (layer B.Cu) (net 12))
 (segment (start 148.75 67.5) (end 150.25 69) (width 1) (layer B.Cu) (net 12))
 (segment (start 148.75 65) (end 148.75 67.5) (width 1) (layer B.Cu) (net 12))
 (segment (start 145.59 61.84) (end 148.75 65) (width 1) (layer B.Cu) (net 12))
 (segment (start 142 64.38) (end 145.38 64.38) (width 1) (layer B.Cu) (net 13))
 (segment (start 156.25 71.75) (end 159 69) (width 1) (layer B.Cu) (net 13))
 (segment (start 150 71.75) (end 156.25 71.75) (width 1) (layer B.Cu) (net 13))
 (segment (start 147 68.75) (end 150 71.75) (width 1) (layer B.Cu) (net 13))
 (segment (start 147 66) (end 147 68.75) (width 1) (layer B.Cu) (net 13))
 (segment (start 145.38 64.38) (end 147 66) (width 1) (layer B.Cu) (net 13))
 (segment (start 142 69.46) (end 145.21 69.46) (width 1) (layer B.Cu) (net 14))
 (segment (start 165.5 71.25) (end 165.5 69) (width 1) (layer B.Cu) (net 14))
 (segment (start 163.25 73.5) (end 165.5 71.25) (width 1) (layer B.Cu) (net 14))
 (segment (start 149.25 73.5) (end 163.25 73.5) (width 1) (layer B.Cu) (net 14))
 (segment (start 145.21 69.46) (end 149.25 73.5) (width 1) (layer B.Cu) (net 14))
 (segment (start 142 72) (end 145.25 72) (width 1) (layer B.Cu) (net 15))
 (segment (start 172 73.25) (end 172 69) (width 1) (layer B.Cu) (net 15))
 (segment (start 170 75.25) (end 172 73.25) (width 1) (layer B.Cu) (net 15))
 (segment (start 148.5 75.25) (end 170 75.25) (width 1) (layer B.Cu) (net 15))
 (segment (start 145.25 72) (end 148.5 75.25) (width 1) (layer B.Cu) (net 15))
 (segment (start 184 75.28) (end 175.97 75.28) (width 1) (layer F.Cu) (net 11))
 (segment (start 152.35 93.85) (end 154.76 93.85) (width 1) (layer F.Cu) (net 11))
 (segment (start 150 91.5) (end 152.35 93.85) (width 1) (layer F.Cu) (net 11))
 (segment (start 150 82.5) (end 150 91.5) (width 1) (layer F.Cu) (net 11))
 (segment (start 152 80.5) (end 150 82.5) (width 1) (layer F.Cu) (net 11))
 (segment (start 170.75 80.5) (end 152 80.5) (width 1) (layer F.Cu) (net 11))
 (segment (start 175.97 75.28) (end 170.75 80.5) (width 1) (layer F.Cu) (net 11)))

